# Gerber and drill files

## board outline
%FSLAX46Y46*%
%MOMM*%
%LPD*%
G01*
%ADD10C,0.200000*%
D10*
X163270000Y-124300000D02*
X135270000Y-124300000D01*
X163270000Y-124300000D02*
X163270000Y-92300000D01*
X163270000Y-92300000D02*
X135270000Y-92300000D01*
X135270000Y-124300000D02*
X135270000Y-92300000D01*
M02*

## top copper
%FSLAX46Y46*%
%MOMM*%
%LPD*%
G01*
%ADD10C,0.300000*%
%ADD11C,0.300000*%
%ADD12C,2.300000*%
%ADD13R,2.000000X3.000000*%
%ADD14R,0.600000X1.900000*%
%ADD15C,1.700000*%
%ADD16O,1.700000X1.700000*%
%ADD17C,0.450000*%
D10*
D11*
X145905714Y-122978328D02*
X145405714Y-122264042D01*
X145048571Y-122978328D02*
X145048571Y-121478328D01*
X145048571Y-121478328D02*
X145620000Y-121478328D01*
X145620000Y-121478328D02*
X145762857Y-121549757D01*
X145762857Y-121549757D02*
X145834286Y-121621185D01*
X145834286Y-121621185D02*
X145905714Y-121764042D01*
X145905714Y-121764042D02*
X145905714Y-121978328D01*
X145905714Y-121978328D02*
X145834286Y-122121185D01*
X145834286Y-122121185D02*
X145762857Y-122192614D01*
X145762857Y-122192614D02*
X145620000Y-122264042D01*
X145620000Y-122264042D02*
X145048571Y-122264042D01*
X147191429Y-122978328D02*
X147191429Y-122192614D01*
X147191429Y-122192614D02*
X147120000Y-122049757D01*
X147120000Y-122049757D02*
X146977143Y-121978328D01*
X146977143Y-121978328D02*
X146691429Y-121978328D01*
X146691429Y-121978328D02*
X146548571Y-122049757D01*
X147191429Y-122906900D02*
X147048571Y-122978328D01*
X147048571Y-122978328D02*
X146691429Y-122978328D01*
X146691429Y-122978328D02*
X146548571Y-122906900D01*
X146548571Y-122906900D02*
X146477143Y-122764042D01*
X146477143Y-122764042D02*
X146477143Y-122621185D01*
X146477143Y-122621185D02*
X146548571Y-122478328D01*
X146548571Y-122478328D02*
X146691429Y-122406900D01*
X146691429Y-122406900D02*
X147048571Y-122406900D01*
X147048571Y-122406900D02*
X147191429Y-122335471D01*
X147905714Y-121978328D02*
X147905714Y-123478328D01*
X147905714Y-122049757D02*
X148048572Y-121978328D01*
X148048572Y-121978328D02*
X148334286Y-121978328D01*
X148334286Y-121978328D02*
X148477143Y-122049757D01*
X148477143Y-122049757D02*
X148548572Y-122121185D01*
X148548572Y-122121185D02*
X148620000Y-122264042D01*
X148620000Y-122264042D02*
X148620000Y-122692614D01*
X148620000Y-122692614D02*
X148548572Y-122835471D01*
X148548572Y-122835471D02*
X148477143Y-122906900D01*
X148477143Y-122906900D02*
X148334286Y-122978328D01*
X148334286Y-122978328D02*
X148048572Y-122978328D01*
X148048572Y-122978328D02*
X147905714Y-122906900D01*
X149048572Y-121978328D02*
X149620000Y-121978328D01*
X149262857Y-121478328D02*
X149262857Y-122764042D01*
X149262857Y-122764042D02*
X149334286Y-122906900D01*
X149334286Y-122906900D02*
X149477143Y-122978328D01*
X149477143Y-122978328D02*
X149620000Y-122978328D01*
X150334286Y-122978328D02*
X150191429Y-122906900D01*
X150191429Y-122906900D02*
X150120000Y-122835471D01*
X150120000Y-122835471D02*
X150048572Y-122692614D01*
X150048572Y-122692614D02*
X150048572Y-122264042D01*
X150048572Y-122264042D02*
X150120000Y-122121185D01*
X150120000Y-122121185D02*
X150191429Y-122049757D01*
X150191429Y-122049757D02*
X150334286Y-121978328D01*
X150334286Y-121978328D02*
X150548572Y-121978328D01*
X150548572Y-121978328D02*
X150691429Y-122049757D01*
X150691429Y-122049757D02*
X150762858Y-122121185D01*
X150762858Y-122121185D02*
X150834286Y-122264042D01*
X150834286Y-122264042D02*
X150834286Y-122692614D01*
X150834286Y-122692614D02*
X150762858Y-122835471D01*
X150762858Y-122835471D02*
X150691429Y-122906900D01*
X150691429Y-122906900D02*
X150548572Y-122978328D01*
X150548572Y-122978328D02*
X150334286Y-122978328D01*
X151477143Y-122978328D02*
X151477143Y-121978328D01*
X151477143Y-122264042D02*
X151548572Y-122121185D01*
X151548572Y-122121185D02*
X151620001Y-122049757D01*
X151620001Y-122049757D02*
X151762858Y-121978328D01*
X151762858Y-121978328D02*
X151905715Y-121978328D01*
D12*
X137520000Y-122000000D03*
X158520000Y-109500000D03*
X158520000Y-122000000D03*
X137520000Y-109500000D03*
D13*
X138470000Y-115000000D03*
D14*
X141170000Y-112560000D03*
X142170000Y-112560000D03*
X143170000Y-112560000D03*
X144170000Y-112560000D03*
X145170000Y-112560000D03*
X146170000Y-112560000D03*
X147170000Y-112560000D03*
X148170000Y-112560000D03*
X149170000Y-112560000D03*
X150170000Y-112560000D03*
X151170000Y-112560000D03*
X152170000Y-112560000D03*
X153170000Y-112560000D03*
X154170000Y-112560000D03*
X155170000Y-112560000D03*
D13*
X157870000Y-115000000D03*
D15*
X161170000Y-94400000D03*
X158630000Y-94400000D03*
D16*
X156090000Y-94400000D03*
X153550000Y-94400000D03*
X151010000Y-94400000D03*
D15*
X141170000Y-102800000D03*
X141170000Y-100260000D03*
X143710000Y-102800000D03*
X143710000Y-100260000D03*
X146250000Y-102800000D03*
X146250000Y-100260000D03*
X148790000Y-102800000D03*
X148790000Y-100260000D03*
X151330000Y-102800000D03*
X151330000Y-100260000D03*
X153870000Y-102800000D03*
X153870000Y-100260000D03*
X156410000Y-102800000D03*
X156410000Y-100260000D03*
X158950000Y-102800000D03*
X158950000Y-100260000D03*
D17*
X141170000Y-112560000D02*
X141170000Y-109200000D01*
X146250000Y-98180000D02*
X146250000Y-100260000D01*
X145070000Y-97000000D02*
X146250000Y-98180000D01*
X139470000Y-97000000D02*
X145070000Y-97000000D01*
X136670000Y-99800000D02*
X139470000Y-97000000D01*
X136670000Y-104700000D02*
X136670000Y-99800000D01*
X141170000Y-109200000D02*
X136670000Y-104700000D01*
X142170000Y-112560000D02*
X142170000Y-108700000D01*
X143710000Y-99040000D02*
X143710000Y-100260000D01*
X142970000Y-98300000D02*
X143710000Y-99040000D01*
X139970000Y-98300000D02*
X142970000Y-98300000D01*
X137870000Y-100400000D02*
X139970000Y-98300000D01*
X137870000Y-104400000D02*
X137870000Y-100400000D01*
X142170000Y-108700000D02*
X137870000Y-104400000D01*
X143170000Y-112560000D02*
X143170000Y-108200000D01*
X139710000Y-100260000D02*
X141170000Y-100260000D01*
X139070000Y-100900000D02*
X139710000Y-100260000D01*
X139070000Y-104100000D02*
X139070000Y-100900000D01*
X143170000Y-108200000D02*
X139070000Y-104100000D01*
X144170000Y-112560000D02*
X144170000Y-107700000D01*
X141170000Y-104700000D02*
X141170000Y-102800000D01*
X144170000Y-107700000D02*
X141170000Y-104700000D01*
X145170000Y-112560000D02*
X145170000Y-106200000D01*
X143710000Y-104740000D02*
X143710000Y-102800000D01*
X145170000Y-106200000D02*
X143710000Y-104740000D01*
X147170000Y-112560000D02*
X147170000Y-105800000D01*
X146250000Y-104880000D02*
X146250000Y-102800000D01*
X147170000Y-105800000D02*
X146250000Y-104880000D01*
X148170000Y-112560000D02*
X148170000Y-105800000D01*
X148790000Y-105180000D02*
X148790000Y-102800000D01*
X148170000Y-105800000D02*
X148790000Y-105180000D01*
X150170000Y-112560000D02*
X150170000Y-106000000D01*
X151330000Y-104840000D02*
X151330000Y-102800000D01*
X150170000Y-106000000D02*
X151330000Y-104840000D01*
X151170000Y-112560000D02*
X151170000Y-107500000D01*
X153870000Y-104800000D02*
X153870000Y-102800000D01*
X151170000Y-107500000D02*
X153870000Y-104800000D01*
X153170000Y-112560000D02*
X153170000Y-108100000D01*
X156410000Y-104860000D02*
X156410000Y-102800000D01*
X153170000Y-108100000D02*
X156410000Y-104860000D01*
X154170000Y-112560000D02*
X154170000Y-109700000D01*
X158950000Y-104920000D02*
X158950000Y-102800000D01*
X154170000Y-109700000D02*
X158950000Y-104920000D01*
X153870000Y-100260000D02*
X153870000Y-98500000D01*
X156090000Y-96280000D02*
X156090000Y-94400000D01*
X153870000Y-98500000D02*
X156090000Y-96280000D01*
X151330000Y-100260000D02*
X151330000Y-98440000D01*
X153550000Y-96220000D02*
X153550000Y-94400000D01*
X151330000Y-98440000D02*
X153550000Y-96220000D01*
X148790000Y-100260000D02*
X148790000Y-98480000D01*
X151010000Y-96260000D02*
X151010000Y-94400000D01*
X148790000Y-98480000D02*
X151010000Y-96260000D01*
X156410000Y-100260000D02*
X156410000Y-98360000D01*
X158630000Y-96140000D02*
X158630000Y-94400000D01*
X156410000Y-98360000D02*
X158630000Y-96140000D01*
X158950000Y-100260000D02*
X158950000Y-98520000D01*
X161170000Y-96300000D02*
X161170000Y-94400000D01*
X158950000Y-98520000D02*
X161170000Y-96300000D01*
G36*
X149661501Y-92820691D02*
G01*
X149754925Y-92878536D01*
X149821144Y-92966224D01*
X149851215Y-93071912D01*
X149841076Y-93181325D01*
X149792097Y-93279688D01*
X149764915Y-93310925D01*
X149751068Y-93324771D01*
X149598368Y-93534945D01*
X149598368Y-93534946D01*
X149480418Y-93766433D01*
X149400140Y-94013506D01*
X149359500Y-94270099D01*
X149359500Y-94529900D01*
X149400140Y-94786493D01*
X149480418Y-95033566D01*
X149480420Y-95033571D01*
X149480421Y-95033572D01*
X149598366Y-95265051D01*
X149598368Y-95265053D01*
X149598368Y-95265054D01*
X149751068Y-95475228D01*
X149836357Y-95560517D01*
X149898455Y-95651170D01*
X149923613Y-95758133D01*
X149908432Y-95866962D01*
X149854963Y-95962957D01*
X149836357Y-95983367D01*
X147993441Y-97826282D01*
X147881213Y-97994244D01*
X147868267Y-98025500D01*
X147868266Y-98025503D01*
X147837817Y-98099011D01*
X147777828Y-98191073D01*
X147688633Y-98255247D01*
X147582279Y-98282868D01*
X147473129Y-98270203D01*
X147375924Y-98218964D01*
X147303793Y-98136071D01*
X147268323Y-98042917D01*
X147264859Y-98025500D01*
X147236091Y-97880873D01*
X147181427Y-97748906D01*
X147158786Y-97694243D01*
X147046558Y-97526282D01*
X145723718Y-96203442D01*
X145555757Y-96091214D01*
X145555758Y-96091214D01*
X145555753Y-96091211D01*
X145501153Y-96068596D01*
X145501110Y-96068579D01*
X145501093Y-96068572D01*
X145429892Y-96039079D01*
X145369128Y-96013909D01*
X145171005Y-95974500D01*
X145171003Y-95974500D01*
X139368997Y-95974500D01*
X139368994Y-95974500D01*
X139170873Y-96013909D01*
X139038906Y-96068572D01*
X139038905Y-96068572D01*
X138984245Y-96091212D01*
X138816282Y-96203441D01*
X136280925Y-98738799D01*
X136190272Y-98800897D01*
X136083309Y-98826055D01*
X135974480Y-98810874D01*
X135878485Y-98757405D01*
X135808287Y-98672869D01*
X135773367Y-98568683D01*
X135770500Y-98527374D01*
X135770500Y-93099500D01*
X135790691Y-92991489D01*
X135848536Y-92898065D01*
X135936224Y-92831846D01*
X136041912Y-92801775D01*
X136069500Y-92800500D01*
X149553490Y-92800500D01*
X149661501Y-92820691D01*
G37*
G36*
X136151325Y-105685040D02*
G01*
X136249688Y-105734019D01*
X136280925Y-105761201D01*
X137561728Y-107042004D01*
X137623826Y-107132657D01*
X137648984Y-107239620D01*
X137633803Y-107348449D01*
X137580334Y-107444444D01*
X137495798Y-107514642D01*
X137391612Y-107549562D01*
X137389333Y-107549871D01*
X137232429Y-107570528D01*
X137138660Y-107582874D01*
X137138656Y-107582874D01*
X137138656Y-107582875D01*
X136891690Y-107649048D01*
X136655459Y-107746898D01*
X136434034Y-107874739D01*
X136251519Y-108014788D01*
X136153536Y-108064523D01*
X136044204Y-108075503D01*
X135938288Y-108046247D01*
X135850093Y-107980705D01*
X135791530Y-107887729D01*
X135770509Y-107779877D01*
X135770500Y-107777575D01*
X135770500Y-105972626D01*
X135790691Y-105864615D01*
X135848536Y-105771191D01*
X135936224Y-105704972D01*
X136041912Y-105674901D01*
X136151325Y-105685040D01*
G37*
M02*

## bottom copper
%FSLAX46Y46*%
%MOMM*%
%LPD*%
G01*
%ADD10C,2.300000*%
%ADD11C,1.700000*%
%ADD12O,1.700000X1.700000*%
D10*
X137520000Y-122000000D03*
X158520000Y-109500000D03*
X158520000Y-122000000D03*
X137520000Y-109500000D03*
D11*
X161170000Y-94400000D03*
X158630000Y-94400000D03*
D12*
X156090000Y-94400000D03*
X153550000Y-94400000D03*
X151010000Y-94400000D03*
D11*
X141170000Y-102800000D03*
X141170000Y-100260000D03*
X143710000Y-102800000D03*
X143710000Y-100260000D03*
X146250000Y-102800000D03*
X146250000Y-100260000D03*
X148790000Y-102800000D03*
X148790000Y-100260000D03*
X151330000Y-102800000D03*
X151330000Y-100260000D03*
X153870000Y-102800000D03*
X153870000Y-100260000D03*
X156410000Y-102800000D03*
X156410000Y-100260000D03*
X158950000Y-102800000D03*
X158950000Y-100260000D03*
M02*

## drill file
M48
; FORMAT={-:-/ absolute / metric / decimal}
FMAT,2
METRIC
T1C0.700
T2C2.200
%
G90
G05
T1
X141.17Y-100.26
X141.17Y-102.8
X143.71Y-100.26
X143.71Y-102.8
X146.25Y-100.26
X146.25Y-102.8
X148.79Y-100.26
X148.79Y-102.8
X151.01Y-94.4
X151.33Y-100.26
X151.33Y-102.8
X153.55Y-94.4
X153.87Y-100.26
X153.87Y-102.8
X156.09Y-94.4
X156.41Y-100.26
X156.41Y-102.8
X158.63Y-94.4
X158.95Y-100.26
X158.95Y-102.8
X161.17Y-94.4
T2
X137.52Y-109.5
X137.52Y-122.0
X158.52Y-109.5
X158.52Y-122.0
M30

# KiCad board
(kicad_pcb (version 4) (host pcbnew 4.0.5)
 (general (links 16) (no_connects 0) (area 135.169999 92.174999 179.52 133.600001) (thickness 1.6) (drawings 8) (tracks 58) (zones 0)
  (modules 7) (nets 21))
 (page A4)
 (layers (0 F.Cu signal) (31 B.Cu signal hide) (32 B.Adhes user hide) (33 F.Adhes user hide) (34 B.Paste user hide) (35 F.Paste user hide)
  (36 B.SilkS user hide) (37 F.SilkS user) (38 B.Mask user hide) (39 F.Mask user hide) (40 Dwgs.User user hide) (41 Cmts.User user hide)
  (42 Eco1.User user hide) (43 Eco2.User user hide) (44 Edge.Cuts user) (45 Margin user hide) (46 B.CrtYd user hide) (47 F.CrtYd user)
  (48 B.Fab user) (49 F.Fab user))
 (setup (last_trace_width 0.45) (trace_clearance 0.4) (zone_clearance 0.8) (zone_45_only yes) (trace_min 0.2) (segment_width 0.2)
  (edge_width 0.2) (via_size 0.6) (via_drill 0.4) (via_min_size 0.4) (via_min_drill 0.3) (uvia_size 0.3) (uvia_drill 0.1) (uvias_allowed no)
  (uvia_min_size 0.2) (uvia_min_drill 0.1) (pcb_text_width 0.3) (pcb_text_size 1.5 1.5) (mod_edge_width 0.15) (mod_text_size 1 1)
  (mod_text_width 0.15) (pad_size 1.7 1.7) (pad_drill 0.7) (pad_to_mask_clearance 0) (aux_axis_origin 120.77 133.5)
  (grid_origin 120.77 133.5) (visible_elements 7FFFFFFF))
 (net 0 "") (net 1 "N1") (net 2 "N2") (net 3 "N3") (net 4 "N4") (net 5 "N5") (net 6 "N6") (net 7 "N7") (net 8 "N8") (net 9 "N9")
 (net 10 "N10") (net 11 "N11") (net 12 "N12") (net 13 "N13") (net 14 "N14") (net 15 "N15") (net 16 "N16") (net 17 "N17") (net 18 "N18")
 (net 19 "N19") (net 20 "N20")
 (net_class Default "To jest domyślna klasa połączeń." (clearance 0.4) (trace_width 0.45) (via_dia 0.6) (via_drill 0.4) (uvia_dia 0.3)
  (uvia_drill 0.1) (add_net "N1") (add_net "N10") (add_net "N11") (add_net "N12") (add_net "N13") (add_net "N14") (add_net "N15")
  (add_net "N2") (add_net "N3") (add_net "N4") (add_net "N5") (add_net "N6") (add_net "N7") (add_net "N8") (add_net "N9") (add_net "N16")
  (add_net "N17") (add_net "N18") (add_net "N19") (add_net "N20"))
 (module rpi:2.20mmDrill (layer F.Cu) (at 137.52 122)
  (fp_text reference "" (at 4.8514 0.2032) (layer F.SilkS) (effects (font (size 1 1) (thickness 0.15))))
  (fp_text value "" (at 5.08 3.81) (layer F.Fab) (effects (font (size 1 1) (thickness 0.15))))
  (pad "" thru_hole circle (at 0 0) (size 2.3 2.3) (drill 2.2) (layers *.Cu *.Mask)))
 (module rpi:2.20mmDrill (layer F.Cu) (at 158.52 109.5)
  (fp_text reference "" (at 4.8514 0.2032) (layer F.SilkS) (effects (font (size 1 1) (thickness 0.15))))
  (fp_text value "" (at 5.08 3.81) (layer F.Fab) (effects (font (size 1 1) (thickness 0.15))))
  (pad "" thru_hole circle (at 0 0) (size 2.3 2.3) (drill 2.2) (layers *.Cu *.Mask)))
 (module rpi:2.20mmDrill (layer F.Cu) (at 158.52 122)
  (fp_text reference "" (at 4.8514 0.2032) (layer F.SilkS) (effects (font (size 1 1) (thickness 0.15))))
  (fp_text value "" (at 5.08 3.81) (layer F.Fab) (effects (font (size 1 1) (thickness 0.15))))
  (pad "" thru_hole circle (at 0 0) (size 2.3 2.3) (drill 2.2) (layers *.Cu *.Mask)))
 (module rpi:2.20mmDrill (layer F.Cu) (at 137.52 109.5)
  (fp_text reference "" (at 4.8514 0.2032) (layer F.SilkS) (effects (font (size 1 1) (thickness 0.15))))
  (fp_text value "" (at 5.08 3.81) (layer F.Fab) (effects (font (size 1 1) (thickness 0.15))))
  (pad "" thru_hole circle (at 0 0) (size 2.3 2.3) (drill 2.2) (layers *.Cu *.Mask)))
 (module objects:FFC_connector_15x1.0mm (layer F.Cu) (at 148.07 115)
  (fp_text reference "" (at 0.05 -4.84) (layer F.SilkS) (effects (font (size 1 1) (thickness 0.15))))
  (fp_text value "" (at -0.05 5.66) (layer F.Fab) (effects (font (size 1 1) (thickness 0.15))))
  (pad "" smd rect (at -9.6 0) (size 2 3) (layers F.Cu F.Paste F.Mask))
  (pad 1 smd rect (at -6.9 -2.44) (size 0.6 1.9) (layers F.Cu F.Paste F.Mask) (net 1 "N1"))
  (pad 2 smd rect (at -5.9 -2.44) (size 0.6 1.9) (layers F.Cu F.Paste F.Mask) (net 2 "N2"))
  (pad 3 smd rect (at -4.9 -2.44) (size 0.6 1.9) (layers F.Cu F.Paste F.Mask) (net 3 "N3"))
  (pad 4 smd rect (at -3.9 -2.44) (size 0.6 1.9) (layers F.Cu F.Paste F.Mask) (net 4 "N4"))
  (pad 5 smd rect (at -2.9 -2.44) (size 0.6 1.9) (layers F.Cu F.Paste F.Mask) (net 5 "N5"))
  (pad 6 smd rect (at -1.9 -2.44) (size 0.6 1.9) (layers F.Cu F.Paste F.Mask) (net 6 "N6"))
  (pad 7 smd rect (at -0.9 -2.44) (size 0.6 1.9) (layers F.Cu F.Paste F.Mask) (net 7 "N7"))
  (pad 8 smd rect (at 0.1 -2.44) (size 0.6 1.9) (layers F.Cu F.Paste F.Mask) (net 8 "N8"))
  (pad 9 smd rect (at 1.1 -2.44) (size 0.6 1.9) (layers F.Cu F.Paste F.Mask) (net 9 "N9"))
  (pad 10 smd rect (at 2.1 -2.44) (size 0.6 1.9) (layers F.Cu F.Paste F.Mask) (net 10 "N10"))
  (pad 11 smd rect (at 3.1 -2.44) (size 0.6 1.9) (layers F.Cu F.Paste F.Mask) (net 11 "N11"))
  (pad 12 smd rect (at 4.1 -2.44) (size 0.6 1.9) (layers F.Cu F.Paste F.Mask) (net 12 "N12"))
  (pad 13 smd rect (at 5.1 -2.44) (size 0.6 1.9) (layers F.Cu F.Paste F.Mask) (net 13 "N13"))
  (pad 14 smd rect (at 6.1 -2.44) (size 0.6 1.9) (layers F.Cu F.Paste F.Mask) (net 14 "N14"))
  (pad 15 smd rect (at 7.1 -2.44) (size 0.6 1.9) (layers F.Cu F.Paste F.Mask) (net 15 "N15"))
  (pad "" smd rect (at 9.8 0) (size 2 3) (layers F.Cu F.Paste F.Mask)))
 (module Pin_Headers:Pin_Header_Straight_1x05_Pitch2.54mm (layer F.Cu) (at 161.17 94.4 270)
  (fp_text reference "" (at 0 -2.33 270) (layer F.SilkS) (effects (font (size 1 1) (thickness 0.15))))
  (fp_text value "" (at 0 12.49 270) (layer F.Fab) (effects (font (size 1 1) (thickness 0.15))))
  (pad 1 thru_hole circle (at 0 0 270) (size 1.7 1.7) (drill 0.7) (layers *.Cu *.Mask) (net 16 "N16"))
  (pad 2 thru_hole circle (at 0 2.54 270) (size 1.7 1.7) (drill 0.7) (layers *.Cu *.Mask) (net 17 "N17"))
  (pad 3 thru_hole oval (at 0 5.08 270) (size 1.7 1.7) (drill 0.7) (layers *.Cu *.Mask) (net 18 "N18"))
  (pad 4 thru_hole oval (at 0 7.62 270) (size 1.7 1.7) (drill 0.7) (layers *.Cu *.Mask) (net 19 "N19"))
  (pad 5 thru_hole oval (at 0 10.16 270) (size 1.7 1.7) (drill 0.7) (layers *.Cu *.Mask) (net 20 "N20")))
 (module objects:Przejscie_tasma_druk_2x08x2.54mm (layer F.Cu) (at 141.17 102.8)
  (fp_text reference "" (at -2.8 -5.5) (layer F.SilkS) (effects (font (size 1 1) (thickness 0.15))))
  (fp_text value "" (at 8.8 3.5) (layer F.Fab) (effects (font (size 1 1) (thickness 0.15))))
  (pad 1 thru_hole circle (at 0 0) (size 1.7 1.7) (drill 0.7) (layers *.Cu *.Mask) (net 4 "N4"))
  (pad 2 thru_hole circle (at 0 -2.54) (size 1.7 1.7) (drill 0.7) (layers *.Cu *.Mask) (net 3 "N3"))
  (pad 3 thru_hole circle (at 2.54 0) (size 1.7 1.7) (drill 0.7) (layers *.Cu *.Mask) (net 5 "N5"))
  (pad 4 thru_hole circle (at 2.54 -2.54) (size 1.7 1.7) (drill 0.7) (layers *.Cu *.Mask) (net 2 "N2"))
  (pad 5 thru_hole circle (at 5.08 0) (size 1.7 1.7) (drill 0.7) (layers *.Cu *.Mask) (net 7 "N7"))
  (pad 6 thru_hole circle (at 5.08 -2.54) (size 1.7 1.7) (drill 0.7) (layers *.Cu *.Mask) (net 1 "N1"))
  (pad 7 thru_hole circle (at 7.62 0) (size 1.7 1.7) (drill 0.7) (layers *.Cu *.Mask) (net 8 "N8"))
  (pad 8 thru_hole circle (at 7.62 -2.54) (size 1.7 1.7) (drill 0.7) (layers *.Cu *.Mask) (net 20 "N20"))
  (pad 9 thru_hole circle (at 10.16 0) (size 1.7 1.7) (drill 0.7) (layers *.Cu *.Mask) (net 10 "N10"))
  (pad 10 thru_hole circle (at 10.16 -2.54) (size 1.7 1.7) (drill 0.7) (layers *.Cu *.Mask) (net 19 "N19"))
  (pad 11 thru_hole circle (at 12.7 0) (size 1.7 1.7) (drill 0.7) (layers *.Cu *.Mask) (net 11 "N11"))
  (pad 12 thru_hole circle (at 12.7 -2.54) (size 1.7 1.7) (drill 0.7) (layers *.Cu *.Mask) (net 18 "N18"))
  (pad 13 thru_hole circle (at 15.24 0) (size 1.7 1.7) (drill 0.7) (layers *.Cu *.Mask) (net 13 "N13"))
  (pad 14 thru_hole circle (at 15.24 -2.54) (size 1.7 1.7) (drill 0.7) (layers *.Cu *.Mask) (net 17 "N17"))
  (pad 15 thru_hole circle (at 17.78 0) (size 1.7 1.7) (drill 0.7) (layers *.Cu *.Mask) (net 14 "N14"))
  (pad 16 thru_hole circle (at 17.78 -2.54) (size 1.7 1.7) (drill 0.7) (layers *.Cu *.Mask) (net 16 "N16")))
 (gr_line (start 163.27 124.3) (end 135.27 124.3) (angle 90) (layer Edge.Cuts) (width 0.2))
 (gr_line (start 163.27 124.3) (end 163.27 92.3) (angle 90) (layer Edge.Cuts) (width 0.2))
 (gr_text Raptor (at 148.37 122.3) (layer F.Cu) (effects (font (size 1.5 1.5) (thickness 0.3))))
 (gr_line (start 163.27 92.3) (end 135.27 92.3) (angle 90) (layer Edge.Cuts) (width 0.2))
 (gr_line (start 135.27 124.3) (end 135.27 92.3) (angle 90) (layer Edge.Cuts) (width 0.2))
 (segment (start 141.17 112.56) (end 141.17 109.2) (width 0.45) (layer F.Cu) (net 1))
 (segment (start 146.25 98.18) (end 146.25 100.26) (width 0.45) (layer F.Cu) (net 1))
 (segment (start 145.07 97) (end 146.25 98.18) (width 0.45) (layer F.Cu) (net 1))
 (segment (start 139.47 97) (end 145.07 97) (width 0.45) (layer F.Cu) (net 1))
 (segment (start 136.67 99.8) (end 139.47 97) (width 0.45) (layer F.Cu) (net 1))
 (segment (start 136.67 104.7) (end 136.67 99.8) (width 0.45) (layer F.Cu) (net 1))
 (segment (start 141.17 109.2) (end 136.67 104.7) (width 0.45) (layer F.Cu) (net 1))
 (segment (start 142.17 112.56) (end 142.17 108.7) (width 0.45) (layer F.Cu) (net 2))
 (segment (start 143.71 99.04) (end 143.71 100.26) (width 0.45) (layer F.Cu) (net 2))
 (segment (start 142.97 98.3) (end 143.71 99.04) (width 0.45) (layer F.Cu) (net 2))
 (segment (start 139.97 98.3) (end 142.97 98.3) (width 0.45) (layer F.Cu) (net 2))
 (segment (start 137.87 100.4) (end 139.97 98.3) (width 0.45) (layer F.Cu) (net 2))
 (segment (start 137.87 104.4) (end 137.87 100.4) (width 0.45) (layer F.Cu) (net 2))
 (segment (start 142.17 108.7) (end 137.87 104.4) (width 0.45) (layer F.Cu) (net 2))
 (segment (start 143.17 112.56) (end 143.17 108.2) (width 0.45) (layer F.Cu) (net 3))
 (segment (start 139.71 100.26) (end 141.17 100.26) (width 0.45) (layer F.Cu) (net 3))
 (segment (start 139.07 100.9) (end 139.71 100.26) (width 0.45) (layer F.Cu) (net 3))
 (segment (start 139.07 104.1) (end 139.07 100.9) (width 0.45) (layer F.Cu) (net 3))
 (segment (start 143.17 108.2) (end 139.07 104.1) (width 0.45) (layer F.Cu) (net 3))
 (segment (start 144.17 112.56) (end 144.17 107.7) (width 0.45) (layer F.Cu) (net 4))
 (segment (start 141.17 104.7) (end 141.17 102.8) (width 0.45) (layer F.Cu) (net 4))
 (segment (start 144.17 107.7) (end 141.17 104.7) (width 0.45) (layer F.Cu) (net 4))
 (segment (start 145.17 112.56) (end 145.17 106.2) (width 0.45) (layer F.Cu) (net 5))
 (segment (start 143.71 104.74) (end 143.71 102.8) (width 0.45) (layer F.Cu) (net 5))
 (segment (start 145.17 106.2) (end 143.71 104.74) (width 0.45) (layer F.Cu) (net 5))
 (segment (start 147.17 112.56) (end 147.17 105.8) (width 0.45) (layer F.Cu) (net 7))
 (segment (start 146.25 104.88) (end 146.25 102.8) (width 0.45) (layer F.Cu) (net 7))
 (segment (start 147.17 105.8) (end 146.25 104.88) (width 0.45) (layer F.Cu) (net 7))
 (segment (start 148.17 112.56) (end 148.17 105.8) (width 0.45) (layer F.Cu) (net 8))
 (segment (start 148.79 105.18) (end 148.79 102.8) (width 0.45) (layer F.Cu) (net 8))
 (segment (start 148.17 105.8) (end 148.79 105.18) (width 0.45) (layer F.Cu) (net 8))
 (segment (start 150.17 112.56) (end 150.17 106) (width 0.45) (layer F.Cu) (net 10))
 (segment (start 151.33 104.84) (end 151.33 102.8) (width 0.45) (layer F.Cu) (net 10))
 (segment (start 150.17 106) (end 151.33 104.84) (width 0.45) (layer F.Cu) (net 10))
 (segment (start 151.17 112.56) (end 151.17 107.5) (width 0.45) (layer F.Cu) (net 11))
 (segment (start 153.87 104.8) (end 153.87 102.8) (width 0.45) (layer F.Cu) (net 11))
 (segment (start 151.17 107.5) (end 153.87 104.8) (width 0.45) (layer F.Cu) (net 11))
 (segment (start 153.17 112.56) (end 153.17 108.1) (width 0.45) (layer F.Cu) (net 13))
 (segment (start 156.41 104.86) (end 156.41 102.8) (width 0.45) (layer F.Cu) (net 13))
 (segment (start 153.17 108.1) (end 156.41 104.86) (width 0.45) (layer F.Cu) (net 13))
 (segment (start 154.17 112.56) (end 154.17 109.7) (width 0.45) (layer F.Cu) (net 14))
 (segment (start 158.95 104.92) (end 158.95 102.8) (width 0.45) (layer F.Cu) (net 14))
 (segment (start 154.17 109.7) (end 158.95 104.92) (width 0.45) (layer F.Cu) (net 14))
 (segment (start 153.87 100.26) (end 153.87 98.5) (width 0.45) (layer F.Cu) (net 18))
 (segment (start 156.09 96.28) (end 156.09 94.4) (width 0.45) (layer F.Cu) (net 18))
 (segment (start 153.87 98.5) (end 156.09 96.28) (width 0.45) (layer F.Cu) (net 18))
 (segment (start 151.33 100.26) (end 151.33 98.44) (width 0.45) (layer F.Cu) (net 19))
 (segment (start 153.55 96.22) (end 153.55 94.4) (width 0.45) (layer F.Cu) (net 19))
 (segment (start 151.33 98.44) (end 153.55 96.22) (width 0.45) (layer F.Cu) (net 19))
 (segment (start 148.79 100.26) (end 148.79 98.48) (width 0.45) (layer F.Cu) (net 20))
 (segment (start 151.01 96.26) (end 151.01 94.4) (width 0.45) (layer F.Cu) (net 20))
 (segment (start 148.79 98.48) (end 151.01 96.26) (width 0.45) (layer F.Cu) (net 20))
 (segment (start 156.41 100.26) (end 156.41 98.36) (width 0.45) (layer F.Cu) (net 17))
 (segment (start 158.63 96.14) (end 158.63 94.4) (width 0.45) (layer F.Cu) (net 17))
 (segment (start 156.41 98.36) (end 158.63 96.14) (width 0.45) (layer F.Cu) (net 17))
 (segment (start 158.95 100.26) (end 158.95 98.52) (width 0.45) (layer F.Cu) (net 16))
 (segment (start 161.17 96.3) (end 161.17 94.4) (width 0.45) (layer F.Cu) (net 16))
 (segment (start 158.95 98.52) (end 161.17 96.3) (width 0.45) (layer F.Cu) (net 16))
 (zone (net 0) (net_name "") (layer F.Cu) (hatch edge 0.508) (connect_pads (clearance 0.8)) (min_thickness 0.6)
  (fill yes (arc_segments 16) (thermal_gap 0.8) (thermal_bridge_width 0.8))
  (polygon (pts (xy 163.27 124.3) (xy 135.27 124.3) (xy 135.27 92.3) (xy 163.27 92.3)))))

